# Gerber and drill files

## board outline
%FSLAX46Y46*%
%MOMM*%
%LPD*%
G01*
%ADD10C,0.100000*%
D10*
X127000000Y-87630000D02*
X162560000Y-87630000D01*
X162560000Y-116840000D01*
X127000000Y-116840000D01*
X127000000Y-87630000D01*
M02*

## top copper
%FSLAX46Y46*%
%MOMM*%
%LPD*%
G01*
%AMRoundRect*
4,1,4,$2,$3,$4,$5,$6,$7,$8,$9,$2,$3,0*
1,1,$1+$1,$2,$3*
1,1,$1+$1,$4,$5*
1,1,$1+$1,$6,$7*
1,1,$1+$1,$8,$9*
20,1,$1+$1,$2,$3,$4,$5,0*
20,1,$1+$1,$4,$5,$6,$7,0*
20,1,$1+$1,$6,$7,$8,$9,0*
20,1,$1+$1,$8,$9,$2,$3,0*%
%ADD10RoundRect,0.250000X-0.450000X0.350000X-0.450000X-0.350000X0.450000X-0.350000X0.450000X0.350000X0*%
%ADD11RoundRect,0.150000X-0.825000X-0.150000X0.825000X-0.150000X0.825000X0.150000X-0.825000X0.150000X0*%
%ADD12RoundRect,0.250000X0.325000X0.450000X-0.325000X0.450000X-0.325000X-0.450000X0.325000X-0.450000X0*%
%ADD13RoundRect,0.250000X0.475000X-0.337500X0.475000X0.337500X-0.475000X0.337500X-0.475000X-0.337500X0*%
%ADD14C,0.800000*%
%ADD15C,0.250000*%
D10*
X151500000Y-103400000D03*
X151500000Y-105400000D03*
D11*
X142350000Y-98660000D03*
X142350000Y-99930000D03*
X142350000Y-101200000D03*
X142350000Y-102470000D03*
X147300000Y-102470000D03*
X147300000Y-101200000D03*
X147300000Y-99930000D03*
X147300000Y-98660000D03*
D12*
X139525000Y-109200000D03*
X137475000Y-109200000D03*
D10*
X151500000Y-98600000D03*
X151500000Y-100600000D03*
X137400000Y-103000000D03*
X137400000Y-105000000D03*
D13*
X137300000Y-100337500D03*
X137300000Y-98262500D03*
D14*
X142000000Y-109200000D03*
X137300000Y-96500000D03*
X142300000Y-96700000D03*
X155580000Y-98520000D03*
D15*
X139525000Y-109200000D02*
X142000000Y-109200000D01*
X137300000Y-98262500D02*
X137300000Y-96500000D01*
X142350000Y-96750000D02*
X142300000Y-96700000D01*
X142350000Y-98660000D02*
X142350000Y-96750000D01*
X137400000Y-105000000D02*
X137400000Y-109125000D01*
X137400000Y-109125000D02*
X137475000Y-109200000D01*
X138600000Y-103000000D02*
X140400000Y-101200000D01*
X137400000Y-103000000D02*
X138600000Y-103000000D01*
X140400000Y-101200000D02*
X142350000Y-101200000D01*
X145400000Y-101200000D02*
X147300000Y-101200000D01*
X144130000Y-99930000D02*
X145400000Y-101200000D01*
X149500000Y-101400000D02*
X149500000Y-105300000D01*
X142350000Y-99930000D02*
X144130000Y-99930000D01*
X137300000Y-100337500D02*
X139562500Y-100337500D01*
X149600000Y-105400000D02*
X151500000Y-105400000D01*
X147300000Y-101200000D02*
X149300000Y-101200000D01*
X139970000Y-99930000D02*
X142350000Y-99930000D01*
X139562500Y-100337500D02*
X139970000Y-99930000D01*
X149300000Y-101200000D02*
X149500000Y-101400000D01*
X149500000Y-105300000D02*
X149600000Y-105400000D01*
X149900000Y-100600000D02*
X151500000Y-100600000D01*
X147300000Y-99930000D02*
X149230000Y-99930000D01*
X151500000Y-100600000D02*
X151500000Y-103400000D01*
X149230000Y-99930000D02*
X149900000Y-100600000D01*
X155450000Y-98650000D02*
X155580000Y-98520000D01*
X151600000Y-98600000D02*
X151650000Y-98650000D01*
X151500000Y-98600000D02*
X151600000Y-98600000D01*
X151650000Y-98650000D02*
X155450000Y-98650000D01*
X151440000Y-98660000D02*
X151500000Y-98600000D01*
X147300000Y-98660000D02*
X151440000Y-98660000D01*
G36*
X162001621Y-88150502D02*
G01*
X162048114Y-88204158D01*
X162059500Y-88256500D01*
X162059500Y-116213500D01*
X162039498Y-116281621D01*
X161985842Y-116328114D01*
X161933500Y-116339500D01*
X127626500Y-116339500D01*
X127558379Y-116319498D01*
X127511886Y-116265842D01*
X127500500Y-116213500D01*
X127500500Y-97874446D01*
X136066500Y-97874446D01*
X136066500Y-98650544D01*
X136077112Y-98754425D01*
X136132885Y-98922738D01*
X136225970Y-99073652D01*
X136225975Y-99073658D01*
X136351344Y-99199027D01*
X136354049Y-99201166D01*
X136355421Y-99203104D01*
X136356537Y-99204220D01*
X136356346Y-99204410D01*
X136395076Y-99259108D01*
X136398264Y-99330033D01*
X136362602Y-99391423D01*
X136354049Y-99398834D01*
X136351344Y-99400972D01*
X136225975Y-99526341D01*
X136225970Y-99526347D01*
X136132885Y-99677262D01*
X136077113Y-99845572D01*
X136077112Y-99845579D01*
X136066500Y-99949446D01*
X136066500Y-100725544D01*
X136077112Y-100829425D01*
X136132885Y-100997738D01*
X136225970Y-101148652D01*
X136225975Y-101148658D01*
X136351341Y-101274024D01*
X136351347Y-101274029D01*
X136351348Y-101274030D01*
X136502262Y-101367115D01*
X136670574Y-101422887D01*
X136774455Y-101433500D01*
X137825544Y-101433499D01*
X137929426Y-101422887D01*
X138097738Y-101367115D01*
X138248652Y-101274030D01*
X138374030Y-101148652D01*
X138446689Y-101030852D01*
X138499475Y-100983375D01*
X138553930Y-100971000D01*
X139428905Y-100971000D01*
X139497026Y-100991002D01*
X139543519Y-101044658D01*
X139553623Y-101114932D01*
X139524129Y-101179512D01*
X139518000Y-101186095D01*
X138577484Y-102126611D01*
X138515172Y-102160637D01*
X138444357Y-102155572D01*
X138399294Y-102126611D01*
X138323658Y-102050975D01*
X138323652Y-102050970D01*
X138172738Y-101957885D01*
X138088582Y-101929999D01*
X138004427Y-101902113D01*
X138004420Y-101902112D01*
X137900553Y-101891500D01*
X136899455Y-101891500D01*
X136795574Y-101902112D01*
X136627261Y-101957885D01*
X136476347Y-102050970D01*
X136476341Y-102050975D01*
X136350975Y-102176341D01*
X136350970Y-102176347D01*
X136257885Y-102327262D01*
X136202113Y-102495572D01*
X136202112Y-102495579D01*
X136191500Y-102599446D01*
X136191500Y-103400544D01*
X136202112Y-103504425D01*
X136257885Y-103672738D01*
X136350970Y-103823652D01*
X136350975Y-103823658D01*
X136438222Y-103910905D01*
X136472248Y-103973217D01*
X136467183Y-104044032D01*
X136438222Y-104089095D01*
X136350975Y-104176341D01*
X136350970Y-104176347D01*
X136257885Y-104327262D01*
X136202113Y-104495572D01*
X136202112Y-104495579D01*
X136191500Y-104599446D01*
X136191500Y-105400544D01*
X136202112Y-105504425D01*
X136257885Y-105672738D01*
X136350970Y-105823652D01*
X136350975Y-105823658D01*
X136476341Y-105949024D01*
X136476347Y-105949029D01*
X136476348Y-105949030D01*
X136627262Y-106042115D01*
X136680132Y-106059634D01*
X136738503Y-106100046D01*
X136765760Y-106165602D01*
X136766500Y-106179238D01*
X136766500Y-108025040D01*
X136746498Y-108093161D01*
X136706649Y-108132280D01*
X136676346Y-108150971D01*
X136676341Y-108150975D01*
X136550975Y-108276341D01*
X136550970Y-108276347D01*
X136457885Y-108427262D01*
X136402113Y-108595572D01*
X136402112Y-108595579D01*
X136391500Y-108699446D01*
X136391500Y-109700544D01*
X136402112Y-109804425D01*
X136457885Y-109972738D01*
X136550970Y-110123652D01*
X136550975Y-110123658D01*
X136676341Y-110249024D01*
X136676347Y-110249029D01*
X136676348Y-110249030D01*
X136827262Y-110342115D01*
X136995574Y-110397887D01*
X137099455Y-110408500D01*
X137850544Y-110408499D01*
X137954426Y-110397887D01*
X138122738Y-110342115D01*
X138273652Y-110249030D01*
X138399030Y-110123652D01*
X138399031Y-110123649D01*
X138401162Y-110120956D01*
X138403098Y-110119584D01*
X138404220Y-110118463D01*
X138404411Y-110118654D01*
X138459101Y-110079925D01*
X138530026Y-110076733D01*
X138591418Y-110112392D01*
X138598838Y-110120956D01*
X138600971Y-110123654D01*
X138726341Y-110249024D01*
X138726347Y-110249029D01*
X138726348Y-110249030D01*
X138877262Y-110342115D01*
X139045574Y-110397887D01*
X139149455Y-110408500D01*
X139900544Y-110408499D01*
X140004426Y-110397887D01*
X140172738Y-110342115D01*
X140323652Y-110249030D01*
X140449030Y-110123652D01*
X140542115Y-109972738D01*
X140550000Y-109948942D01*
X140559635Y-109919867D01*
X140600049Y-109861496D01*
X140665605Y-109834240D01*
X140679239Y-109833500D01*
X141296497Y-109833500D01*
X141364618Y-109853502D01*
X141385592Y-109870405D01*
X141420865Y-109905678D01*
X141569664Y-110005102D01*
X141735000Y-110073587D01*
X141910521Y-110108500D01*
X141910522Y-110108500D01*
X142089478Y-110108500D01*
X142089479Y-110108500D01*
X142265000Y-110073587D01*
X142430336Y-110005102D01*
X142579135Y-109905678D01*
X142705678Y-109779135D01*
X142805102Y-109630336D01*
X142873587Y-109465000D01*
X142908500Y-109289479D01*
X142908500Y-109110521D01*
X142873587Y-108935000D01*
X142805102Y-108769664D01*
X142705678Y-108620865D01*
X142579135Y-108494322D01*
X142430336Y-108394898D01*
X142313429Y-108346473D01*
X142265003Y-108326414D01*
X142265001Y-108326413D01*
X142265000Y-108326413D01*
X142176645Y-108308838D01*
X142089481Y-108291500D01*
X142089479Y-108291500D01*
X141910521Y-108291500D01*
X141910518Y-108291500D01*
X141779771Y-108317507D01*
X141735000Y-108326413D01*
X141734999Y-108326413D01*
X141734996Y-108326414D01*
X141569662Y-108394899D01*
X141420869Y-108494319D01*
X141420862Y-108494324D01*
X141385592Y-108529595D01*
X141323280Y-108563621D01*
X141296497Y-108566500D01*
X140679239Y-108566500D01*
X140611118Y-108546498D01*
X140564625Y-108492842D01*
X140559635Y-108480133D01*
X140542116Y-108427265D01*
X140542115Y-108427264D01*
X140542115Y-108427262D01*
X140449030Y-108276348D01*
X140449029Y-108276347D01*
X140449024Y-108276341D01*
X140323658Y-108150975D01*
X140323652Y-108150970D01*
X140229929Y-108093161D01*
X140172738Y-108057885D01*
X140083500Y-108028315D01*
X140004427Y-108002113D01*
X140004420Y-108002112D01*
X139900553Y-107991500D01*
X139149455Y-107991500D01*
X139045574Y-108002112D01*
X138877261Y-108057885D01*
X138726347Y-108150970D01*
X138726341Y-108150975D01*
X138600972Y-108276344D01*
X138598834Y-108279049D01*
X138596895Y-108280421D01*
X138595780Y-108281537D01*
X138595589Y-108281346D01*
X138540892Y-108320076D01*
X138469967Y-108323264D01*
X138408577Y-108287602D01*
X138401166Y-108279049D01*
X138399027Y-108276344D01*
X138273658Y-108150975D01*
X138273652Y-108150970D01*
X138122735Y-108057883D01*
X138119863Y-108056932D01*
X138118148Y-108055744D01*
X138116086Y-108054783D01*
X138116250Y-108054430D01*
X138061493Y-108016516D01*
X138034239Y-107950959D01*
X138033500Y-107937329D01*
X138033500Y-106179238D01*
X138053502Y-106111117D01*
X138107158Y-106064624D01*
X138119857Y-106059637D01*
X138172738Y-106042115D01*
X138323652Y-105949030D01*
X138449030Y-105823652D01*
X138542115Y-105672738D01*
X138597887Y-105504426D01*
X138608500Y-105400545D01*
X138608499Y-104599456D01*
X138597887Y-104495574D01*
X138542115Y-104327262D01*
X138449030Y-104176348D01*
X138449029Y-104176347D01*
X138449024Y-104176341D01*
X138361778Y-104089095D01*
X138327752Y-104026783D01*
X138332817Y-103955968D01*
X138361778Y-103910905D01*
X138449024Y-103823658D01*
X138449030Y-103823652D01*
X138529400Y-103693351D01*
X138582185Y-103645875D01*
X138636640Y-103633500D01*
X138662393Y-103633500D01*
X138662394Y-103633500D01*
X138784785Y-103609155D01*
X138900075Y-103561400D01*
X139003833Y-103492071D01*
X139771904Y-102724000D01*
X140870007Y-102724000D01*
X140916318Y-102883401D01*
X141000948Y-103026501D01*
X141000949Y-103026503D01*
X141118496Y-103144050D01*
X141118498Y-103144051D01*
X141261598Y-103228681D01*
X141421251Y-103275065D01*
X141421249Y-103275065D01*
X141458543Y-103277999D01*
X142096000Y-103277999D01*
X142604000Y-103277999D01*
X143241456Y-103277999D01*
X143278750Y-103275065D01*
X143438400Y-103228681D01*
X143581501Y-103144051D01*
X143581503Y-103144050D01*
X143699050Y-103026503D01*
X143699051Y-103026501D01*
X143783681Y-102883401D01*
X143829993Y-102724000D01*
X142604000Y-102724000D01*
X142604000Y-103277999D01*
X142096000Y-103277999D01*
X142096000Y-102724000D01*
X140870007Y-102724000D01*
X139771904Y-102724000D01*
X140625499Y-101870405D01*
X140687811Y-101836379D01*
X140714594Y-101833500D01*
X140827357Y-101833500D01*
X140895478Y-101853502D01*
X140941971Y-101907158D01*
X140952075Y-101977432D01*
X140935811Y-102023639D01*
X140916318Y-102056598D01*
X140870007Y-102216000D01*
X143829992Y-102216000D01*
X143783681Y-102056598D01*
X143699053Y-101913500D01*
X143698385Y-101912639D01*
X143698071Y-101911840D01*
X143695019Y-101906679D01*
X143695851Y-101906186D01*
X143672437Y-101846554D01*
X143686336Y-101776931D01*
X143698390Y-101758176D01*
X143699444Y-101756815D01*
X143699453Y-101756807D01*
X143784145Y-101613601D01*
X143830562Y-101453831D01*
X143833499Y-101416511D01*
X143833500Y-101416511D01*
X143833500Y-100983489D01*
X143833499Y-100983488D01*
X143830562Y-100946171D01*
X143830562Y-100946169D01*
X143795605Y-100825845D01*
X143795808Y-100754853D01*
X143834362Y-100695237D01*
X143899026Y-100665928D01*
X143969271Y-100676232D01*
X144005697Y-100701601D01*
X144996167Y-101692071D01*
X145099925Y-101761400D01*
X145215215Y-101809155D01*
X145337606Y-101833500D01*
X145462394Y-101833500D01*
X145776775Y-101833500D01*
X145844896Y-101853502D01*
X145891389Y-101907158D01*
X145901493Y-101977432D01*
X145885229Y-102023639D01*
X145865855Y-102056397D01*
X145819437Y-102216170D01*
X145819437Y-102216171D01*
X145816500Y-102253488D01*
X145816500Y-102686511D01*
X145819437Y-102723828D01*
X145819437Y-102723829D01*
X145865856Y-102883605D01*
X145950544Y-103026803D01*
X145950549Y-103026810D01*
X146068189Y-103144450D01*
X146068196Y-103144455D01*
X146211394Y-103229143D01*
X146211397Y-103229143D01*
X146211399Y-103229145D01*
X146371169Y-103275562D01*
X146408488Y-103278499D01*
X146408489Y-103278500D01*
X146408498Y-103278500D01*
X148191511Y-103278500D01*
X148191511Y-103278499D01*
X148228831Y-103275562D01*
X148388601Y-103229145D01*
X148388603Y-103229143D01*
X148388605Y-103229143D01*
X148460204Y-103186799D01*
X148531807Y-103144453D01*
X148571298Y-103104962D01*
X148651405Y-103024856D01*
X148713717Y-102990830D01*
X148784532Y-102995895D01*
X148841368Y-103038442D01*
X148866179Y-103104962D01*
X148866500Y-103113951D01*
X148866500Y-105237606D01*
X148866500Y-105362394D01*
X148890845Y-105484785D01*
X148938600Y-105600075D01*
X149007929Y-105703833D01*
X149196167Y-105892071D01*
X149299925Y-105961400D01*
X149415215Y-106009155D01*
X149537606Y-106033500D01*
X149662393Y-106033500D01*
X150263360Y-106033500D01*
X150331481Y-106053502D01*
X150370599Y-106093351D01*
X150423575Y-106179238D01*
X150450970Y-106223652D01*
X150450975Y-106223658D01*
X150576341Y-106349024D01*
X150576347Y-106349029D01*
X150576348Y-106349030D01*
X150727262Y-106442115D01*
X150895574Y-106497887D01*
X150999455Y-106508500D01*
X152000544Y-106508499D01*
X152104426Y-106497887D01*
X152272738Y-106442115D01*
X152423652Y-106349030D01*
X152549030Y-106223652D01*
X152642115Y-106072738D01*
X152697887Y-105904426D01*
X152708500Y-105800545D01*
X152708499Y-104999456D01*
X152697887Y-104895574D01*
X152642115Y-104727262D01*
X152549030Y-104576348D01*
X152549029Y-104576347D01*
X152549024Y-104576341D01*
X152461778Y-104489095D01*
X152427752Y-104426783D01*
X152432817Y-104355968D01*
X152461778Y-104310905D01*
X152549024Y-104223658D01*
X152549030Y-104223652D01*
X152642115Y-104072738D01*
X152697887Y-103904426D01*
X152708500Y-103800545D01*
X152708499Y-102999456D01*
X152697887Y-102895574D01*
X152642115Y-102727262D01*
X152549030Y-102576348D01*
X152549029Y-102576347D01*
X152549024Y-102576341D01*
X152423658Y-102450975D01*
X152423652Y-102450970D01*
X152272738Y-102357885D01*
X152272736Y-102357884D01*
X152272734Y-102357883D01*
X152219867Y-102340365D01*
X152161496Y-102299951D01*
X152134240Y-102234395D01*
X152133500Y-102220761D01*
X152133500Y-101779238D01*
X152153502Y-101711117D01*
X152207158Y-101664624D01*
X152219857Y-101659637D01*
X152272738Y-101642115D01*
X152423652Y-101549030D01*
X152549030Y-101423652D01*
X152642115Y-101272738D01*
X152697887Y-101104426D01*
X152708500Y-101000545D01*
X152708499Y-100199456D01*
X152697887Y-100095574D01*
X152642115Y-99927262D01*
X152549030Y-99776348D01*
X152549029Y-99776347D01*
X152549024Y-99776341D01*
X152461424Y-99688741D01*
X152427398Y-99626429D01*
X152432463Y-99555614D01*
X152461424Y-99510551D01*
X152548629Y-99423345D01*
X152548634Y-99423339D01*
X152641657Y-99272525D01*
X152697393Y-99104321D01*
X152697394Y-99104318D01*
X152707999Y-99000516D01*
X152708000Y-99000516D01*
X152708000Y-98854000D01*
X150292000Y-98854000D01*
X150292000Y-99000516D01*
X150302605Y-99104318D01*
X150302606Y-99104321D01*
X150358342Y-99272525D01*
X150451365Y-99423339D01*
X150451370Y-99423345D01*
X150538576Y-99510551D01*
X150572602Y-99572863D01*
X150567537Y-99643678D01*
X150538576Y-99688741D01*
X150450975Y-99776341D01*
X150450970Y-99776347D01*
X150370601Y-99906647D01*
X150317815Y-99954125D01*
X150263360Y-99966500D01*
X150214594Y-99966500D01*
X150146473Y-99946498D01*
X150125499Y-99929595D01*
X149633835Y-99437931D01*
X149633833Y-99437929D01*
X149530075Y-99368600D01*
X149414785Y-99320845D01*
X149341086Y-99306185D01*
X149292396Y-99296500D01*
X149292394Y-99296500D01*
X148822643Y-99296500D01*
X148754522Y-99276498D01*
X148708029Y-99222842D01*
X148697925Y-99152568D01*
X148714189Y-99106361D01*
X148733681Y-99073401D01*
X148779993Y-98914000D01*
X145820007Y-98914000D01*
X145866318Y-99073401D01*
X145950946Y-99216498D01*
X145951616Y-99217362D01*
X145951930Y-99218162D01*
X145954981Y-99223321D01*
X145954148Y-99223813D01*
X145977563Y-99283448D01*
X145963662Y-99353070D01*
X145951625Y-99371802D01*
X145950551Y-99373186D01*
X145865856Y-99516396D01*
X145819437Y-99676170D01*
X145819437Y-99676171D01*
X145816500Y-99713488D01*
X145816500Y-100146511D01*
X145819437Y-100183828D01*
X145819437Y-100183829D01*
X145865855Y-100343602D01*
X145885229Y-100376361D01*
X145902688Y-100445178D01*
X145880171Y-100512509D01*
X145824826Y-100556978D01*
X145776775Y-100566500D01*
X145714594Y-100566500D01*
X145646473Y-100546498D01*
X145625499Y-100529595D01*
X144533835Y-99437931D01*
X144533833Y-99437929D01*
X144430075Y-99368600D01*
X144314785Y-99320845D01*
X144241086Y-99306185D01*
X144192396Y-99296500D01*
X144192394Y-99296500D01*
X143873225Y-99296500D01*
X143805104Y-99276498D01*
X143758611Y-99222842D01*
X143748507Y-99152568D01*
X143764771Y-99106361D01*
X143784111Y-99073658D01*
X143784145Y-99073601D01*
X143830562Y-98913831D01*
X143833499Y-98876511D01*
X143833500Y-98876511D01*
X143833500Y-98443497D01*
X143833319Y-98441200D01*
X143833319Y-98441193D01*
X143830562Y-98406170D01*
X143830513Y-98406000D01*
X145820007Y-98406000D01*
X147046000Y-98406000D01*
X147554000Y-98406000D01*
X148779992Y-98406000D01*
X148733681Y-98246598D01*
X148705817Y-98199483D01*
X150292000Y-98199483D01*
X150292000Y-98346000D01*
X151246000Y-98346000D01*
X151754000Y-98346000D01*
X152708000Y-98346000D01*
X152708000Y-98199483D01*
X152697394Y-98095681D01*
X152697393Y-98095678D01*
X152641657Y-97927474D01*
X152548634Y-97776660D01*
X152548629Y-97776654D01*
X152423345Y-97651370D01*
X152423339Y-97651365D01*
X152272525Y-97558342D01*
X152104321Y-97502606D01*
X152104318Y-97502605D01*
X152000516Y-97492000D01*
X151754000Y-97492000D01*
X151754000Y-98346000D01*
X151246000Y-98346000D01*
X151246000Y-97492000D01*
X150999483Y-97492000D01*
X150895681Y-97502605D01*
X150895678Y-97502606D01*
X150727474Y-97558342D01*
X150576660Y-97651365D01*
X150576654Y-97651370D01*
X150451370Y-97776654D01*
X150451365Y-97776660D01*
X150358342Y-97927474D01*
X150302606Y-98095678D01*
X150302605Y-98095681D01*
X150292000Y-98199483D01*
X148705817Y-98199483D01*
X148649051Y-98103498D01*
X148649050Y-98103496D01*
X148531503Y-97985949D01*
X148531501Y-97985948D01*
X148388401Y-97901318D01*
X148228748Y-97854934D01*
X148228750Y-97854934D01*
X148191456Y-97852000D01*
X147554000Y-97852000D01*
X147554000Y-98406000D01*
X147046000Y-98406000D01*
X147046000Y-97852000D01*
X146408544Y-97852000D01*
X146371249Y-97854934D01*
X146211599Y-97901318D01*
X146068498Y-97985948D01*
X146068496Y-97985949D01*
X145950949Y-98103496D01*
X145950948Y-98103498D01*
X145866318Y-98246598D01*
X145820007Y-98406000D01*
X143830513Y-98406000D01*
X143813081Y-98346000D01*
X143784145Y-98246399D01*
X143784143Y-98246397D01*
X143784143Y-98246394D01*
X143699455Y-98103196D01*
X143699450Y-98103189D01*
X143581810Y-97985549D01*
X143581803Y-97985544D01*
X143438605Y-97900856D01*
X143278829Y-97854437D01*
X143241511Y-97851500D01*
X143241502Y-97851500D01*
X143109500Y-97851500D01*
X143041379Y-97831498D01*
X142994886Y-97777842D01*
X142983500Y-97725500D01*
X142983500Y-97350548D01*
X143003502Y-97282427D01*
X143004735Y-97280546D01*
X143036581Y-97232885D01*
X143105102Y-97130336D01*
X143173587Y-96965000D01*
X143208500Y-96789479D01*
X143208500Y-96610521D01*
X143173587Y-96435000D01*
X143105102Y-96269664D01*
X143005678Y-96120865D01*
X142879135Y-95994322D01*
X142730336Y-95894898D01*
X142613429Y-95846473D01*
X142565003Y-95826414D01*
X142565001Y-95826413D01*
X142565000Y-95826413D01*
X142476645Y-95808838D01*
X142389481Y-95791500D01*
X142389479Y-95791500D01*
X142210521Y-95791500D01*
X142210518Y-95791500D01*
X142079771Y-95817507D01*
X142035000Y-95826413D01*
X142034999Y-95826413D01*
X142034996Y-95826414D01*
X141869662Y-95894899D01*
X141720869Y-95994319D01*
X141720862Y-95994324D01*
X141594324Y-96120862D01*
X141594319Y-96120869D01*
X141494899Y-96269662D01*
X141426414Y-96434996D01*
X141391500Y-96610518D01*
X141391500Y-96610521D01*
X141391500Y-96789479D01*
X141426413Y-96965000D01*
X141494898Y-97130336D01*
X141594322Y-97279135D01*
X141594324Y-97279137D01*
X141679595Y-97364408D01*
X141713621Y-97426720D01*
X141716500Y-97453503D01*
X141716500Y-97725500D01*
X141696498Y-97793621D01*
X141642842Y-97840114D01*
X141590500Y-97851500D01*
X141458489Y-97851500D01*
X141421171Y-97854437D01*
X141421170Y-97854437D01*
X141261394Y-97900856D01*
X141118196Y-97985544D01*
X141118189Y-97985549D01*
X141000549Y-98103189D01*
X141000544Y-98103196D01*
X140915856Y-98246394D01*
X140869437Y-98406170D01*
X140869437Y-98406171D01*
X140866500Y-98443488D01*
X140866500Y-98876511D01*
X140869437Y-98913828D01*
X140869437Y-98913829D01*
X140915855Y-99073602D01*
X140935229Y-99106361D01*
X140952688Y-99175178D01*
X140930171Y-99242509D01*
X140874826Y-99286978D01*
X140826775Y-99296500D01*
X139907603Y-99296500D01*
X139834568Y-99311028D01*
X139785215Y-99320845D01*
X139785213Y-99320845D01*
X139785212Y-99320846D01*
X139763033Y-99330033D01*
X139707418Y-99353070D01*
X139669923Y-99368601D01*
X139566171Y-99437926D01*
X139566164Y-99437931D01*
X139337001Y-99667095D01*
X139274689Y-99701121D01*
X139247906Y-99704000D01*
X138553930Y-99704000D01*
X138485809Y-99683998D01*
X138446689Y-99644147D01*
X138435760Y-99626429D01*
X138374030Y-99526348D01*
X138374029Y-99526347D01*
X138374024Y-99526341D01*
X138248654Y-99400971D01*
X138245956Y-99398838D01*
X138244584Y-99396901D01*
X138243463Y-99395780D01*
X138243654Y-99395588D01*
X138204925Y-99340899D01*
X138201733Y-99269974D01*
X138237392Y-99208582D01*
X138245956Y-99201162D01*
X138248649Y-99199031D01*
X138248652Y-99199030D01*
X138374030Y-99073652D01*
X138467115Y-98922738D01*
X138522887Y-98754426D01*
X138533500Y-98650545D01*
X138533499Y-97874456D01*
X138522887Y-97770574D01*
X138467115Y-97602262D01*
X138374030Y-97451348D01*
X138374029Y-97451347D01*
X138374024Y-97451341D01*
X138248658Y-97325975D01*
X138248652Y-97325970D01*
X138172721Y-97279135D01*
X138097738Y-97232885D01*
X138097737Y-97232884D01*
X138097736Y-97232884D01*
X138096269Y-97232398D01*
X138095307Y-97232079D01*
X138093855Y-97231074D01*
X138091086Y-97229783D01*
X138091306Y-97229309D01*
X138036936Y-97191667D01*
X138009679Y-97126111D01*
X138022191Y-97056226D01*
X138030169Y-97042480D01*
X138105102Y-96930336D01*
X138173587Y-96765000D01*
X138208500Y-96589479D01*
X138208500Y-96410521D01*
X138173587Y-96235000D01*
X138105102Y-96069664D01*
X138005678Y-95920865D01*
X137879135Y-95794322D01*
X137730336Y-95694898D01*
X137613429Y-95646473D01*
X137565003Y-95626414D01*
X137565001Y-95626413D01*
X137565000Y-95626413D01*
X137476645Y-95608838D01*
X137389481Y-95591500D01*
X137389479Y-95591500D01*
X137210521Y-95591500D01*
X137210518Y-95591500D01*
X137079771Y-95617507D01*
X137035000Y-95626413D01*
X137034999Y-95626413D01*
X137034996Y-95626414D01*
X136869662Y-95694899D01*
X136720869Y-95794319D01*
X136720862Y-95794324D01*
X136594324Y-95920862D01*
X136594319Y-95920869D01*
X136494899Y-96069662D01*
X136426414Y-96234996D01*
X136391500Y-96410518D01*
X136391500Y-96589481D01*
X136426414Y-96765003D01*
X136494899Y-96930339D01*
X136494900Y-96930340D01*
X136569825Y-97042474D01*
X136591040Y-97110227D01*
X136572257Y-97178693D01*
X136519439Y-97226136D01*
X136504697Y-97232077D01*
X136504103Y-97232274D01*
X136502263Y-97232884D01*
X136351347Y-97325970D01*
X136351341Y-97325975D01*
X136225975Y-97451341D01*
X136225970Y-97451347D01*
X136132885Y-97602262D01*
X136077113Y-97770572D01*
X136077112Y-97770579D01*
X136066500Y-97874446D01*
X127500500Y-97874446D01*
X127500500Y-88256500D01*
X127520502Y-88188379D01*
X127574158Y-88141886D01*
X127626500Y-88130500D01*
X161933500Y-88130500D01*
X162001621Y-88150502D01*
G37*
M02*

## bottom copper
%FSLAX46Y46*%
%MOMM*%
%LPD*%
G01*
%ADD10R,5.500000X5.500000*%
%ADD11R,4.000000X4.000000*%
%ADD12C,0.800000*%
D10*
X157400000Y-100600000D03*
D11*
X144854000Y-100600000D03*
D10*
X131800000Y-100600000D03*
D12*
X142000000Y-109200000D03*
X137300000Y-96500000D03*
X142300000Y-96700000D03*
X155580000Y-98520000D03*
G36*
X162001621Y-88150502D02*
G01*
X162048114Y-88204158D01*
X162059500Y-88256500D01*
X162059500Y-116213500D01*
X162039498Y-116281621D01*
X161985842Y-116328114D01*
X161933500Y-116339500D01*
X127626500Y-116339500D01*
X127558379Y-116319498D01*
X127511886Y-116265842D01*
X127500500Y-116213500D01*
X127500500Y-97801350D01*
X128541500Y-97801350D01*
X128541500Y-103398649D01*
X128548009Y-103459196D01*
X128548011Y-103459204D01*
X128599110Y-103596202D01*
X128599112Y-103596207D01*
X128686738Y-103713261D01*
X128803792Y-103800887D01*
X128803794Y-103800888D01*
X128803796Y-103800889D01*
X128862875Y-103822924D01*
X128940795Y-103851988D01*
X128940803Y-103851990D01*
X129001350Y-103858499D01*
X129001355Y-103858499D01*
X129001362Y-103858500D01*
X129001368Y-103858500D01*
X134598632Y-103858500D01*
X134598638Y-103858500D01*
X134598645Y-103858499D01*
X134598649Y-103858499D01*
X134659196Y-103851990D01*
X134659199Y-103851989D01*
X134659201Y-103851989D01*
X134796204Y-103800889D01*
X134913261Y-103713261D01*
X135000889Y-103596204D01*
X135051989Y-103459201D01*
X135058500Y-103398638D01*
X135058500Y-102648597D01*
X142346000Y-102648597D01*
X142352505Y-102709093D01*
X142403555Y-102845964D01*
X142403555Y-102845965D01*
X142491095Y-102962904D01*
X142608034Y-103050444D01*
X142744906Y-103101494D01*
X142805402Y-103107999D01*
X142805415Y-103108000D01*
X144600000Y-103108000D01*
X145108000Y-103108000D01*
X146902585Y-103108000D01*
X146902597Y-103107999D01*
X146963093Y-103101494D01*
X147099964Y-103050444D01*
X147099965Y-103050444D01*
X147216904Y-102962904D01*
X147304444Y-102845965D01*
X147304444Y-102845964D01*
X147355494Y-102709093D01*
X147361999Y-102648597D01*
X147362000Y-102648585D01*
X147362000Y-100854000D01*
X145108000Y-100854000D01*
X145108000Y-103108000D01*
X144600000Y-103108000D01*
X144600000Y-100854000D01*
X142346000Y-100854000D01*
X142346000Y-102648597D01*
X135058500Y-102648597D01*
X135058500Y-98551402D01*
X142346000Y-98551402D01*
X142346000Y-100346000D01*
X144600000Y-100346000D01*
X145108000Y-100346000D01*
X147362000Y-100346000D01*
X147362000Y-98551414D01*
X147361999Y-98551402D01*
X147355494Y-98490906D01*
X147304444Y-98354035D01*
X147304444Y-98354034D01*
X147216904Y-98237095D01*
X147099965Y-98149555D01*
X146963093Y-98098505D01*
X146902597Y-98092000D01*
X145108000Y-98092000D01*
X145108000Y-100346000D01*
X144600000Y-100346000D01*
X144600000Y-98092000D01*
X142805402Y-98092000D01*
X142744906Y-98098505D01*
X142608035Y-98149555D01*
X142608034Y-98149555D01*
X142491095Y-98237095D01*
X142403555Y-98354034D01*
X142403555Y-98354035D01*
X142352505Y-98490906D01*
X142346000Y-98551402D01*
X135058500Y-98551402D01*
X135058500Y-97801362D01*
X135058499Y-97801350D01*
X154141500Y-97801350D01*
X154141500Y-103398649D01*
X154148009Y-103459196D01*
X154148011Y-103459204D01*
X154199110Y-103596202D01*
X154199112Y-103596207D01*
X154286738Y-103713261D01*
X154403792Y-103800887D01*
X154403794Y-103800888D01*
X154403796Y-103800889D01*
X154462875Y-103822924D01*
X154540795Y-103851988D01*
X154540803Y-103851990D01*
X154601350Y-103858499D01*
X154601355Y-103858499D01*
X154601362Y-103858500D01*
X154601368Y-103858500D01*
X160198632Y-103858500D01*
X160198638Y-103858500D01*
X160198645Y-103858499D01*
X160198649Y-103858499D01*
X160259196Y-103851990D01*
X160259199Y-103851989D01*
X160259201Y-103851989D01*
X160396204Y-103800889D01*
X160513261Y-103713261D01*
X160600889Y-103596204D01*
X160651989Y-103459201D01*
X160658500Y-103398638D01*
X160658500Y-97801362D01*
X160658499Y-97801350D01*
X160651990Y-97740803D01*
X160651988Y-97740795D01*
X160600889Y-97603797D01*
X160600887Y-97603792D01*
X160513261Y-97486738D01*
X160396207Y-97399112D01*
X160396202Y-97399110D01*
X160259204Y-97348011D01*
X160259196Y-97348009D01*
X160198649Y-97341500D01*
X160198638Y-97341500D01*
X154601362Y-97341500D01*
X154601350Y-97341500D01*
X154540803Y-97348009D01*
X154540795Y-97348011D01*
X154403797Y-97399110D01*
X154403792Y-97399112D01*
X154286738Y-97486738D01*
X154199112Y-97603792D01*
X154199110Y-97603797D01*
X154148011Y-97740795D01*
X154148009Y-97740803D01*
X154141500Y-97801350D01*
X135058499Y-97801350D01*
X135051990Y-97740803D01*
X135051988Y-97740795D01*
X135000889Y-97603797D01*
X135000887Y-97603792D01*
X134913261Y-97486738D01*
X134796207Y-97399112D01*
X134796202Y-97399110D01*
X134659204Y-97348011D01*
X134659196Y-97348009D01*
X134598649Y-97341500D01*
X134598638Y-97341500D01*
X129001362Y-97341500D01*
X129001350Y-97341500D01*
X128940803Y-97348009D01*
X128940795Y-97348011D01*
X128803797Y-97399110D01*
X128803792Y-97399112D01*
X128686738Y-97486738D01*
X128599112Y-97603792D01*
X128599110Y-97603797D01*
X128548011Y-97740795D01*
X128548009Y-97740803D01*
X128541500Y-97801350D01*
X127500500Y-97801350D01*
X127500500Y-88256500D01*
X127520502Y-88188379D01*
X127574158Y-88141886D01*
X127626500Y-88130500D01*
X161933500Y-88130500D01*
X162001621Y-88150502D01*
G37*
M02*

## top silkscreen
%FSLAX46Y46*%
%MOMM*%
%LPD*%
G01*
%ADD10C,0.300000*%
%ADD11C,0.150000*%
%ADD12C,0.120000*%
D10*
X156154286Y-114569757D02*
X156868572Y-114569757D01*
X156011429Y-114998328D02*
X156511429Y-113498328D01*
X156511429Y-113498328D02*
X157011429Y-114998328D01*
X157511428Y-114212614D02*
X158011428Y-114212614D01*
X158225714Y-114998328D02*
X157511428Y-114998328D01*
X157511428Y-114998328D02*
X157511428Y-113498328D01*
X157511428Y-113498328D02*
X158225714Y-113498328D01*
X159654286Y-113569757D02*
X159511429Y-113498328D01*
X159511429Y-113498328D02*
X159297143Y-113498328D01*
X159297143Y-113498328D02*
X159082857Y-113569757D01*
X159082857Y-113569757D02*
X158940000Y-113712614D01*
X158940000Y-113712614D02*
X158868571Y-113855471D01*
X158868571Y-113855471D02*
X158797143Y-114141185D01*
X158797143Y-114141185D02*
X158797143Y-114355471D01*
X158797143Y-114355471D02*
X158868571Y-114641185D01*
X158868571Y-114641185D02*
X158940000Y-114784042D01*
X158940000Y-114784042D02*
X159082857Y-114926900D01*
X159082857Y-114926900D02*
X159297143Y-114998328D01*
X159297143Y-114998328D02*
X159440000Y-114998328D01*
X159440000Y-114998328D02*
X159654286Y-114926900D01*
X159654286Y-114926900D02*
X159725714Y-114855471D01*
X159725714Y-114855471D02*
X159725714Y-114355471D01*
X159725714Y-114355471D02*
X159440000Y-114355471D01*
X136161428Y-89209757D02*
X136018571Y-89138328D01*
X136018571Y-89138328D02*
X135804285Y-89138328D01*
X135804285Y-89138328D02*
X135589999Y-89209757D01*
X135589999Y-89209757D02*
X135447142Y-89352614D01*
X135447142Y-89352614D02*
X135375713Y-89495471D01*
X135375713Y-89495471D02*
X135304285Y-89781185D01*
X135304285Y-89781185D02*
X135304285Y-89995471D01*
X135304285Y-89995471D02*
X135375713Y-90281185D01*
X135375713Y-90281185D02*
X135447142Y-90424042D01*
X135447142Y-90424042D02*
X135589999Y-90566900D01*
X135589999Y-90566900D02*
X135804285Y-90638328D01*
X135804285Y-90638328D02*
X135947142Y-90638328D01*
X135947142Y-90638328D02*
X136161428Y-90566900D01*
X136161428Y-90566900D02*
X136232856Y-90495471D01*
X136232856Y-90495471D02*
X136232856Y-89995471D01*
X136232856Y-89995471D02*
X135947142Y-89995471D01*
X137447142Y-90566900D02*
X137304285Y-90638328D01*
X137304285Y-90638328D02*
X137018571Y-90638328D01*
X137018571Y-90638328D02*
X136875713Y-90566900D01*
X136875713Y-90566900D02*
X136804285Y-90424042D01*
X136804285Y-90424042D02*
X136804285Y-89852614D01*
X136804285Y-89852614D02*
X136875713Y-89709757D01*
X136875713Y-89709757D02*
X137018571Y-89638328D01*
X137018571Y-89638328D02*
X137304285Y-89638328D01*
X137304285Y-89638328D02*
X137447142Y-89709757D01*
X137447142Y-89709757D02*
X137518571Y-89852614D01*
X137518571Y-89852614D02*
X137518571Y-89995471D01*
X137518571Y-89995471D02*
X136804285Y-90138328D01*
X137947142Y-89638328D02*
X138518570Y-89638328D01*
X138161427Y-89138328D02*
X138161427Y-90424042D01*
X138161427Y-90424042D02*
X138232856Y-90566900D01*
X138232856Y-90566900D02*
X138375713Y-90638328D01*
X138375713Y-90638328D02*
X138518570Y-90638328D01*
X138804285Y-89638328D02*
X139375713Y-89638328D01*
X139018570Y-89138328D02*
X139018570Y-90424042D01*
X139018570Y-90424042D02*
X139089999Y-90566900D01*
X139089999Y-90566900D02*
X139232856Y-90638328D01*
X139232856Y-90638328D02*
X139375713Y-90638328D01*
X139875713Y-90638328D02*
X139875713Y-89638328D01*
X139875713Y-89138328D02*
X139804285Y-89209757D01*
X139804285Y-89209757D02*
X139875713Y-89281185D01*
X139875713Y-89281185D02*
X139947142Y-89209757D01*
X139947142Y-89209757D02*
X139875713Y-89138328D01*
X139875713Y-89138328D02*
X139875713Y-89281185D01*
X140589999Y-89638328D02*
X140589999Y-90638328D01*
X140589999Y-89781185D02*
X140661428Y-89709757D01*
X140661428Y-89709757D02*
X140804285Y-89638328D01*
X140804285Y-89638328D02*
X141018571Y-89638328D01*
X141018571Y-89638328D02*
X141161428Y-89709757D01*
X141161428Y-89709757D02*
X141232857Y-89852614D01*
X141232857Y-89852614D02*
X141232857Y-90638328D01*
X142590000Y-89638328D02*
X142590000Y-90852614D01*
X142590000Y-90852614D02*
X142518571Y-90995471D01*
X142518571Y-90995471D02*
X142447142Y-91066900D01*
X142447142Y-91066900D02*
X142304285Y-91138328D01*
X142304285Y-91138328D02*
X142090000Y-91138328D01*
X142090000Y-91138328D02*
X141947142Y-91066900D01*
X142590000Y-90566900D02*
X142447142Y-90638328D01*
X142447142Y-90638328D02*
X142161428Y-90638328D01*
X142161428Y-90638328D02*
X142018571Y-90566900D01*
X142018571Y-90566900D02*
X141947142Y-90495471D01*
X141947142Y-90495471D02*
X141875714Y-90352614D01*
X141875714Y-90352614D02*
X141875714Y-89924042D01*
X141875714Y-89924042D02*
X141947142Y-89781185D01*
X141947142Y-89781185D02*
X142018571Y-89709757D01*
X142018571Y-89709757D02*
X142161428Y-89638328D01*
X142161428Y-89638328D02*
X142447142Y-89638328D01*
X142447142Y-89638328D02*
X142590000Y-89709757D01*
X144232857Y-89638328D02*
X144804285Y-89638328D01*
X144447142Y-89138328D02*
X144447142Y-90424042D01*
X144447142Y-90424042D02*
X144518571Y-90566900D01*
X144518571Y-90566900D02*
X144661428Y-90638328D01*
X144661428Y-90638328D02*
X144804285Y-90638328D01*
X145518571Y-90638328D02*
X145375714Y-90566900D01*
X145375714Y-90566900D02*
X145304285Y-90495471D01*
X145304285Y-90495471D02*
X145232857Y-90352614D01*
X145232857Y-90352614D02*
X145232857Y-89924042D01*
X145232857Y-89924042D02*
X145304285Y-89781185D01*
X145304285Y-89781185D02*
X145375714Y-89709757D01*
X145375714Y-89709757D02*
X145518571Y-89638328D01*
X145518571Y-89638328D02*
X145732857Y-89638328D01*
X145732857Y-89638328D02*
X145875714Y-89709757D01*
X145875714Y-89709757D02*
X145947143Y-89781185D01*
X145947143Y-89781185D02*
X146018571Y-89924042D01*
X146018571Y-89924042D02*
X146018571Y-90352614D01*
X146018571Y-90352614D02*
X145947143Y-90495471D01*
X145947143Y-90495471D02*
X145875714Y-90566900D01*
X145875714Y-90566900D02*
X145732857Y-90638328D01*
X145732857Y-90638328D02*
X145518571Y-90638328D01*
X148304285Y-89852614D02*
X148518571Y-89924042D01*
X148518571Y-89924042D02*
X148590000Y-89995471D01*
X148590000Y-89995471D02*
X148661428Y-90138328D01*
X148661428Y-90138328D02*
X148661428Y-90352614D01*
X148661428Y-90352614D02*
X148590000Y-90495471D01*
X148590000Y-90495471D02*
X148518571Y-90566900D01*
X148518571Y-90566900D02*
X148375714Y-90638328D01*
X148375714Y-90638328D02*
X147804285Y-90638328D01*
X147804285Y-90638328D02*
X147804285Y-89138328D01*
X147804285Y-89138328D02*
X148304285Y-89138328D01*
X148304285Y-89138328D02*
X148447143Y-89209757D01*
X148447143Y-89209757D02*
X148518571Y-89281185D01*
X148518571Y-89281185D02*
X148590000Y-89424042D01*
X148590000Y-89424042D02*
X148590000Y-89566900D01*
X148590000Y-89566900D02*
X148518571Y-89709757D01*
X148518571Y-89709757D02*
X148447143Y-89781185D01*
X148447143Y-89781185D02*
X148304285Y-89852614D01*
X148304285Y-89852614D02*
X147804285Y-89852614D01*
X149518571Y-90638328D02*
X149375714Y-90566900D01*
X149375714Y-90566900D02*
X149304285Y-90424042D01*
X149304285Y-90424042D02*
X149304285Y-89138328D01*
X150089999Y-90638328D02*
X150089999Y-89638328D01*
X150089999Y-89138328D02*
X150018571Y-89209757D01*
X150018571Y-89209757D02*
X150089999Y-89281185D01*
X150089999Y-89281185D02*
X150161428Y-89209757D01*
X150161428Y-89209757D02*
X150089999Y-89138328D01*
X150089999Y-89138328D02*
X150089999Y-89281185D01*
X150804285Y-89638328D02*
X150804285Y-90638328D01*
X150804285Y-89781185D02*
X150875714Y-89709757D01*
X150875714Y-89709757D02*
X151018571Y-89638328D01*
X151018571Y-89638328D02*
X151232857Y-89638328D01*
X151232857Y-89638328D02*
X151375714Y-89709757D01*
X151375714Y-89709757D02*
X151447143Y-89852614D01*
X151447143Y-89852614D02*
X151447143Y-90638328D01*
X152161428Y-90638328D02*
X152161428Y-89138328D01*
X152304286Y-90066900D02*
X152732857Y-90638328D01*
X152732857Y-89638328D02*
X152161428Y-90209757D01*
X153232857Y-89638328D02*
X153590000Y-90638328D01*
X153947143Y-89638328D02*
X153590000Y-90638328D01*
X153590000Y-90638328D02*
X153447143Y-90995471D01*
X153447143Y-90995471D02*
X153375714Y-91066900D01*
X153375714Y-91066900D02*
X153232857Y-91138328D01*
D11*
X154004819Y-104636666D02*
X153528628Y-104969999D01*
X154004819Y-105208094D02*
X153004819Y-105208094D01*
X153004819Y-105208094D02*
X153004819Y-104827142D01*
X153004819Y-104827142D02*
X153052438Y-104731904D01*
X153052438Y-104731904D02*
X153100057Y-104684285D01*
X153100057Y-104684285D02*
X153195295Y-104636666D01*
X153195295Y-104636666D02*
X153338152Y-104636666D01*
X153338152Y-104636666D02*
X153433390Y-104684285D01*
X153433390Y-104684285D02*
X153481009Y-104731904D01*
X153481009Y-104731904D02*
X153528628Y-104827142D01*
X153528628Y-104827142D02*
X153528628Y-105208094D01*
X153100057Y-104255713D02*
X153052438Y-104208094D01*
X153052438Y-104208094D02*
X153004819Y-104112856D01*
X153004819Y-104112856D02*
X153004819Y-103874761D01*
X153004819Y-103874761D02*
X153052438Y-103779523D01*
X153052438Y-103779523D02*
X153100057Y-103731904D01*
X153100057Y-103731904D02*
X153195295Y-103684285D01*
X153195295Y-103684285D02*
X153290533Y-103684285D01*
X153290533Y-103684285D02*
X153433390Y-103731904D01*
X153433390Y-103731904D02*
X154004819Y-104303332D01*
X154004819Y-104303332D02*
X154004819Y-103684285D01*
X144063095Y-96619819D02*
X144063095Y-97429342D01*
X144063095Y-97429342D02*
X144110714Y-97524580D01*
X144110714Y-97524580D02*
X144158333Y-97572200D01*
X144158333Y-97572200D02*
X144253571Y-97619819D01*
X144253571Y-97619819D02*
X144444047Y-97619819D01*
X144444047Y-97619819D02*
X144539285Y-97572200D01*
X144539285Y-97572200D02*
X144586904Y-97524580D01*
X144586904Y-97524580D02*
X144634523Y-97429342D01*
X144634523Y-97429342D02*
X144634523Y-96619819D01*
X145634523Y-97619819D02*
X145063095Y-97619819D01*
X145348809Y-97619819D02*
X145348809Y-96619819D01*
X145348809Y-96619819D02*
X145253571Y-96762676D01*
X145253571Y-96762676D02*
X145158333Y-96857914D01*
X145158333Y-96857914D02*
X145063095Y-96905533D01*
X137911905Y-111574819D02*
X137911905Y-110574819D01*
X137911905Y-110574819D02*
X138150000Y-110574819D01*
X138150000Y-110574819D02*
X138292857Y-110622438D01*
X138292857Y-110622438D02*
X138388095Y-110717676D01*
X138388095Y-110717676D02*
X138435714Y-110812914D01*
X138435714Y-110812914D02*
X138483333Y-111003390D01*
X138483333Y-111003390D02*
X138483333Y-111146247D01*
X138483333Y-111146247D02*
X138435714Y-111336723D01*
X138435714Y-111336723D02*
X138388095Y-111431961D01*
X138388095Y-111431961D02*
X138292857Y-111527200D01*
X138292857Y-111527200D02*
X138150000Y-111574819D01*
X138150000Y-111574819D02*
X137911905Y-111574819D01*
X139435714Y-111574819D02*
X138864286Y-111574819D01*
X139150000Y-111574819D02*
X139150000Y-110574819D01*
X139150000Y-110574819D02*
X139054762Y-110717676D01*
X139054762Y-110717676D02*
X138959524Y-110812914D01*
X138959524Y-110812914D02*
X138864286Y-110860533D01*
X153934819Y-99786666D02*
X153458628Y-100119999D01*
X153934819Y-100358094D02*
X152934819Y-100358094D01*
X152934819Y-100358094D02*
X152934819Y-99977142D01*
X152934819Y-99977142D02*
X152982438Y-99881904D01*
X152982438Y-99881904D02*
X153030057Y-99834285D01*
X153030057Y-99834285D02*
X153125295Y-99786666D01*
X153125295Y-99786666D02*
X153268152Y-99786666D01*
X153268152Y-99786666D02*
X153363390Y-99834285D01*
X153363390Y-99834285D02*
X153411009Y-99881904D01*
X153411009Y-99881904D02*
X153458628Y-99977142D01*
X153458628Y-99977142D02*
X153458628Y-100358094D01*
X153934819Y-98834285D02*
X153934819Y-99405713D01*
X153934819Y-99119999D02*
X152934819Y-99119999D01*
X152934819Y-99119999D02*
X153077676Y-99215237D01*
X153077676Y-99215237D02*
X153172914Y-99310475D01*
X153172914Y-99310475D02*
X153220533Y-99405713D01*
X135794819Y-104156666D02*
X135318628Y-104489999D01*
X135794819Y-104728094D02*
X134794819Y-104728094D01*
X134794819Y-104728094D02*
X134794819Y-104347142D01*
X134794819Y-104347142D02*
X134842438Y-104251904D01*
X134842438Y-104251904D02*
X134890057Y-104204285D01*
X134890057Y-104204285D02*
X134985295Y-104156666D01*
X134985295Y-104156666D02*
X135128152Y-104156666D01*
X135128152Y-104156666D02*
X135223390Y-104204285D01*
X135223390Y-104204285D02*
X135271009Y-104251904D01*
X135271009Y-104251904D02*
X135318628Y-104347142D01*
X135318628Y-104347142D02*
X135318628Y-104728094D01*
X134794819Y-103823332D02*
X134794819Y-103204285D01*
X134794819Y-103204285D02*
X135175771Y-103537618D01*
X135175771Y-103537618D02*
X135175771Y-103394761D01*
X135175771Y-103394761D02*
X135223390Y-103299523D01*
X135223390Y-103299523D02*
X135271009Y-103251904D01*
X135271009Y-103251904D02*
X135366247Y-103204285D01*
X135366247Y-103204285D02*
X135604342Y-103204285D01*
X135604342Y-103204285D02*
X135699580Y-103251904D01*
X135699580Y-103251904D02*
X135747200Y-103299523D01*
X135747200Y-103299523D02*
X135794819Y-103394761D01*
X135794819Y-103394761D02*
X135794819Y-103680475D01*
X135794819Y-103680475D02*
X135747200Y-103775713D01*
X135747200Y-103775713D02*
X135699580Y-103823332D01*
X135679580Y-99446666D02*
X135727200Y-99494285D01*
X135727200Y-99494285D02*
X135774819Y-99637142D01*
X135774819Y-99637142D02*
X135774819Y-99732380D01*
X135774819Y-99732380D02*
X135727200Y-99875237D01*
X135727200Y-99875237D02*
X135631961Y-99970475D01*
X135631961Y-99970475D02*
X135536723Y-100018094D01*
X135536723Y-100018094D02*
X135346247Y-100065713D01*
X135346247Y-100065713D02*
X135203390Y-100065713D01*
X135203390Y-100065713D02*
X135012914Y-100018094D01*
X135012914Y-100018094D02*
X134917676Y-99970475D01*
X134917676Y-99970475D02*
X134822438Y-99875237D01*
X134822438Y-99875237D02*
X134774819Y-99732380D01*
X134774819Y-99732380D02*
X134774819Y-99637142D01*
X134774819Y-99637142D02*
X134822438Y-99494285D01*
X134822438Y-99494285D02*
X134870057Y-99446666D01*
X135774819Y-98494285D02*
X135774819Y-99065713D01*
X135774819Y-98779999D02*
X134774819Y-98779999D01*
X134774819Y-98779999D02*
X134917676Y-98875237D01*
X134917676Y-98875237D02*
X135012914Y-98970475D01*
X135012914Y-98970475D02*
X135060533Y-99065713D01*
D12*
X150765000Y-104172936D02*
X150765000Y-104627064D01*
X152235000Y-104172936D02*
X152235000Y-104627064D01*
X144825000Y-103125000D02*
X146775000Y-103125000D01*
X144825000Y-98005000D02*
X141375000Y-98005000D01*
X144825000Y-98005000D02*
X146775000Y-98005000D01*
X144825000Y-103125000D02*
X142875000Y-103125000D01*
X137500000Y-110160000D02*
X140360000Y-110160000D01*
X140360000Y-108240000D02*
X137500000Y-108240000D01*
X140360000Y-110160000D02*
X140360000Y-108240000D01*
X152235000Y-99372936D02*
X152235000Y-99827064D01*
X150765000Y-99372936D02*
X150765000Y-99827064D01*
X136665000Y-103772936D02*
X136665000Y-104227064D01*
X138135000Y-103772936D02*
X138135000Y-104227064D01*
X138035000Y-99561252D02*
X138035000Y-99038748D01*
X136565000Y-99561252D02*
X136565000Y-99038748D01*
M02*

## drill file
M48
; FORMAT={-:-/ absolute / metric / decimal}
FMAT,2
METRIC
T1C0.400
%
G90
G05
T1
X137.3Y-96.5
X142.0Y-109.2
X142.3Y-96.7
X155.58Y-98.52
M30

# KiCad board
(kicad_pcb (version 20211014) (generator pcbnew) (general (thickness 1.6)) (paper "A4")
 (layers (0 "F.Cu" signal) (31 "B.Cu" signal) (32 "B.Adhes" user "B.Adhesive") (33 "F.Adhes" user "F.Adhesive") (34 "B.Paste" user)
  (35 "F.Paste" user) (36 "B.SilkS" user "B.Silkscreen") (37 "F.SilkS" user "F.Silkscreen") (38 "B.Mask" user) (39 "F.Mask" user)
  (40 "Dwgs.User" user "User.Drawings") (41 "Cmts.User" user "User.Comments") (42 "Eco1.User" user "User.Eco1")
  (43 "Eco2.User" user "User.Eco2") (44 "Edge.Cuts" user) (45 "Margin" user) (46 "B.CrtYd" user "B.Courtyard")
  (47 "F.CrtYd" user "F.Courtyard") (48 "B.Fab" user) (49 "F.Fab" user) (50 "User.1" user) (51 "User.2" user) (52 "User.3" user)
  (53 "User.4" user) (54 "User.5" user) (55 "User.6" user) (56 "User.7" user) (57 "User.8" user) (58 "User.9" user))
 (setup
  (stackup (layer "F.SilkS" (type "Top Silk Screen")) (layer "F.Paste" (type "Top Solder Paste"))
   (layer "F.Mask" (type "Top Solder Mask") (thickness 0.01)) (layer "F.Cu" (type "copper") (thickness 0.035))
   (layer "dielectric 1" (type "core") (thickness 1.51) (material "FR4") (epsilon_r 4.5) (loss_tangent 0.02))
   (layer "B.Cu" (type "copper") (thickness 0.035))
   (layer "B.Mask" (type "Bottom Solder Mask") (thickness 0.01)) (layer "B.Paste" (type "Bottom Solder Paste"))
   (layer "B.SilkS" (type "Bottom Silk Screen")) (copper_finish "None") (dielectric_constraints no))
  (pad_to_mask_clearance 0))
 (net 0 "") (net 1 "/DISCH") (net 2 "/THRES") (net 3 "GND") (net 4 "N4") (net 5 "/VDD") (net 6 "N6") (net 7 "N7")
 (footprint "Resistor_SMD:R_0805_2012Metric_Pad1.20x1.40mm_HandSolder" (layer "F.Cu") (at 151.5 104.4 -90)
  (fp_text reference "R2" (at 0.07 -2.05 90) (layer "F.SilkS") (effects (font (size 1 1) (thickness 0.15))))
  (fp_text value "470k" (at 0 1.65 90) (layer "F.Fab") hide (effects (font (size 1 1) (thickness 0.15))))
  (fp_line (start -0.227064 0.735) (end 0.227064 0.735) (layer "F.SilkS") (width 0.12))
  (fp_line (start -0.227064 -0.735) (end 0.227064 -0.735) (layer "F.SilkS") (width 0.12))
  (pad "1" smd roundrect (at -1 0 270) (size 1.2 1.4) (layers "F.Cu" "F.Paste" "F.Mask") (roundrect_rratio 0.208333) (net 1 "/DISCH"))
  (pad "2" smd roundrect (at 1 0 270) (size 1.2 1.4) (layers "F.Cu" "F.Paste" "F.Mask") (roundrect_rratio 0.208333) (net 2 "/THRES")))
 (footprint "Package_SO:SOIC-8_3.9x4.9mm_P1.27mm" (layer "F.Cu") (at 144.825 100.565)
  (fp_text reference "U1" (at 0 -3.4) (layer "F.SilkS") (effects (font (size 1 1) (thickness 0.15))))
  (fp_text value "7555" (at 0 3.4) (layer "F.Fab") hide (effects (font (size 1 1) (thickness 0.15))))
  (fp_line (start 0 2.56) (end 1.95 2.56) (layer "F.SilkS") (width 0.12))
  (fp_line (start 0 -2.56) (end -3.45 -2.56) (layer "F.SilkS") (width 0.12))
  (fp_line (start 0 -2.56) (end 1.95 -2.56) (layer "F.SilkS") (width 0.12))
  (fp_line (start 0 2.56) (end -1.95 2.56) (layer "F.SilkS") (width 0.12))
  (pad "1" smd roundrect (at -2.475 -1.905) (size 1.95 0.6) (layers "F.Cu" "F.Paste" "F.Mask") (roundrect_rratio 0.25) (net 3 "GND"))
  (pad "2" smd roundrect (at -2.475 -0.635) (size 1.95 0.6) (layers "F.Cu" "F.Paste" "F.Mask") (roundrect_rratio 0.25) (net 2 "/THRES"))
  (pad "3" smd roundrect (at -2.475 0.635) (size 1.95 0.6) (layers "F.Cu" "F.Paste" "F.Mask") (roundrect_rratio 0.25) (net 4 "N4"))
  (pad "4" smd roundrect (at -2.475 1.905) (size 1.95 0.6) (layers "F.Cu" "F.Paste" "F.Mask") (roundrect_rratio 0.25) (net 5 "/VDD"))
  (pad "5" smd roundrect (at 2.475 1.905) (size 1.95 0.6) (layers "F.Cu" "F.Paste" "F.Mask") (roundrect_rratio 0.25) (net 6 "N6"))
  (pad "6" smd roundrect (at 2.475 0.635) (size 1.95 0.6) (layers "F.Cu" "F.Paste" "F.Mask") (roundrect_rratio 0.25) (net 2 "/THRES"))
  (pad "7" smd roundrect (at 2.475 -0.635) (size 1.95 0.6) (layers "F.Cu" "F.Paste" "F.Mask") (roundrect_rratio 0.25) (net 1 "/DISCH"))
  (pad "8" smd roundrect (at 2.475 -1.905) (size 1.95 0.6) (layers "F.Cu" "F.Paste" "F.Mask") (roundrect_rratio 0.25) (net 5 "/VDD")))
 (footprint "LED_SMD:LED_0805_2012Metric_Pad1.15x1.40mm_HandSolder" (layer "F.Cu") (at 138.5 109.2 180)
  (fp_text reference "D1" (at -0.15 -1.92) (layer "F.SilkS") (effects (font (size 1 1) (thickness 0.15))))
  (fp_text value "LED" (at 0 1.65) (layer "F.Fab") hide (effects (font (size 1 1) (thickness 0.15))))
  (fp_line (start 1 -0.96) (end -1.86 -0.96) (layer "F.SilkS") (width 0.12))
  (fp_line (start -1.86 0.96) (end 1 0.96) (layer "F.SilkS") (width 0.12))
  (fp_line (start -1.86 -0.96) (end -1.86 0.96) (layer "F.SilkS") (width 0.12))
  (pad "1" smd roundrect (at -1.025 0 180) (size 1.15 1.4) (layers "F.Cu" "F.Paste" "F.Mask") (roundrect_rratio 0.217391) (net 3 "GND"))
  (pad "2" smd roundrect (at 1.025 0 180) (size 1.15 1.4) (layers "F.Cu" "F.Paste" "F.Mask") (roundrect_rratio 0.217391) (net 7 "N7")))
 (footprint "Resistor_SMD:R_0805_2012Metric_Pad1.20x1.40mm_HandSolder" (layer "F.Cu") (at 151.5 99.6 -90)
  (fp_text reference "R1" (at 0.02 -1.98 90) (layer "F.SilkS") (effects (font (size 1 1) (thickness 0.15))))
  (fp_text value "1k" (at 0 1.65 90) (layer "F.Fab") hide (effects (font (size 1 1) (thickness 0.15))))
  (fp_line (start -0.227064 -0.735) (end 0.227064 -0.735) (layer "F.SilkS") (width 0.12))
  (fp_line (start -0.227064 0.735) (end 0.227064 0.735) (layer "F.SilkS") (width 0.12))
  (pad "1" smd roundrect (at -1 0 270) (size 1.2 1.4) (layers "F.Cu" "F.Paste" "F.Mask") (roundrect_rratio 0.208333) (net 5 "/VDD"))
  (pad "2" smd roundrect (at 1 0 270) (size 1.2 1.4) (layers "F.Cu" "F.Paste" "F.Mask") (roundrect_rratio 0.208333) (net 1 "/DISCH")))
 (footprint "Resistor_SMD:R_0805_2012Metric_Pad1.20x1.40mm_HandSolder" (layer "F.Cu") (at 137.4 104 -90)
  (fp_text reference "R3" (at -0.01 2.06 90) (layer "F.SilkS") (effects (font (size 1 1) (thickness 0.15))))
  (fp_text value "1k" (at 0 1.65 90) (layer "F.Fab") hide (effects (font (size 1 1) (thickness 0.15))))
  (fp_line (start -0.227064 0.735) (end 0.227064 0.735) (layer "F.SilkS") (width 0.12))
  (fp_line (start -0.227064 -0.735) (end 0.227064 -0.735) (layer "F.SilkS") (width 0.12))
  (pad "1" smd roundrect (at -1 0 270) (size 1.2 1.4) (layers "F.Cu" "F.Paste" "F.Mask") (roundrect_rratio 0.208333) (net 4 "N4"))
  (pad "2" smd roundrect (at 1 0 270) (size 1.2 1.4) (layers "F.Cu" "F.Paste" "F.Mask") (roundrect_rratio 0.208333) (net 7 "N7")))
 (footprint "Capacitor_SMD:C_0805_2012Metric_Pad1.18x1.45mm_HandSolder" (layer "F.Cu") (at 137.3 99.3 90)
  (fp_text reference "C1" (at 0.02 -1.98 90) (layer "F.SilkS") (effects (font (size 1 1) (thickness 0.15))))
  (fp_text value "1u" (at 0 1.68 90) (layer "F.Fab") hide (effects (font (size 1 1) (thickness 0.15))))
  (fp_line (start -0.261252 0.735) (end 0.261252 0.735) (layer "F.SilkS") (width 0.12))
  (fp_line (start -0.261252 -0.735) (end 0.261252 -0.735) (layer "F.SilkS") (width 0.12))
  (pad "1" smd roundrect (at -1.0375 0 90) (size 1.175 1.45) (layers "F.Cu" "F.Paste" "F.Mask") (roundrect_rratio 0.212766) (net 2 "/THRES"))
  (pad "2" smd roundrect (at 1.0375 0 90) (size 1.175 1.45) (layers "F.Cu" "F.Paste" "F.Mask") (roundrect_rratio 0.212766) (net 3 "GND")))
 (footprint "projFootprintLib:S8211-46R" (layer "B.Cu") (at 144.6 100.6 180)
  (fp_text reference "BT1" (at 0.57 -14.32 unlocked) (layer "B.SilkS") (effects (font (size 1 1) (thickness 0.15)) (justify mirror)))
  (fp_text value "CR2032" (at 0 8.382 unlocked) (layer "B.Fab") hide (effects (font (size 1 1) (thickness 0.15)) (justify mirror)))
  (pad "1" smd rect (at -12.8 0 180) (size 5.5 5.5) (layers "B.Cu" "B.Paste" "B.Mask") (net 5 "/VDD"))
  (pad "2" smd rect (at -0.254 0 180) (size 4 4) (layers "B.Cu" "B.Paste" "B.Mask") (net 3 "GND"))
  (pad "3" smd rect (at 12.8 0 180) (size 5.5 5.5) (layers "B.Cu" "B.Paste" "B.Mask")))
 (gr_rect (start 127 87.63) (end 162.56 116.84) (layer "Edge.Cuts") (width 0.1) (fill none))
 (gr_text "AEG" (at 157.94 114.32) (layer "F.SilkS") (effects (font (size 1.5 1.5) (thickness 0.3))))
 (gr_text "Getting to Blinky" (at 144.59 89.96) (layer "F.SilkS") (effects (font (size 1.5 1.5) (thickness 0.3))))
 (segment (start 139.525 109.2) (end 142 109.2) (width 0.25) (layer "F.Cu") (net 3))
 (segment (start 137.3 98.2625) (end 137.3 96.5) (width 0.25) (layer "F.Cu") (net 3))
 (segment (start 142.35 96.75) (end 142.3 96.7) (width 0.25) (layer "F.Cu") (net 3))
 (segment (start 142.35 98.66) (end 142.35 96.75) (width 0.25) (layer "F.Cu") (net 3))
 (via (at 142 109.2) (size 0.8) (drill 0.4) (layers "F.Cu" "B.Cu") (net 3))
 (via (at 137.3 96.5) (size 0.8) (drill 0.4) (layers "F.Cu" "B.Cu") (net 3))
 (via (at 142.3 96.7) (size 0.8) (drill 0.4) (layers "F.Cu" "B.Cu") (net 3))
 (segment (start 137.4 105) (end 137.4 109.125) (width 0.25) (layer "F.Cu") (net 7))
 (segment (start 137.4 109.125) (end 137.475 109.2) (width 0.25) (layer "F.Cu") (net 7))
 (segment (start 138.6 103) (end 140.4 101.2) (width 0.25) (layer "F.Cu") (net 4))
 (segment (start 137.4 103) (end 138.6 103) (width 0.25) (layer "F.Cu") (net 4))
 (segment (start 140.4 101.2) (end 142.35 101.2) (width 0.25) (layer "F.Cu") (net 4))
 (segment (start 145.4 101.2) (end 147.3 101.2) (width 0.25) (layer "F.Cu") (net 2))
 (segment (start 144.13 99.93) (end 145.4 101.2) (width 0.25) (layer "F.Cu") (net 2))
 (segment (start 149.5 101.4) (end 149.5 105.3) (width 0.25) (layer "F.Cu") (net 2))
 (segment (start 142.35 99.93) (end 144.13 99.93) (width 0.25) (layer "F.Cu") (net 2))
 (segment (start 137.3 100.3375) (end 139.5625 100.3375) (width 0.25) (layer "F.Cu") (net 2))
 (segment (start 149.6 105.4) (end 151.5 105.4) (width 0.25) (layer "F.Cu") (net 2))
 (segment (start 147.3 101.2) (end 149.3 101.2) (width 0.25) (layer "F.Cu") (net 2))
 (segment (start 139.97 99.93) (end 142.35 99.93) (width 0.25) (layer "F.Cu") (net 2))
 (segment (start 139.5625 100.3375) (end 139.97 99.93) (width 0.25) (layer "F.Cu") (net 2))
 (segment (start 149.3 101.2) (end 149.5 101.4) (width 0.25) (layer "F.Cu") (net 2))
 (segment (start 149.5 105.3) (end 149.6 105.4) (width 0.25) (layer "F.Cu") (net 2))
 (segment (start 149.9 100.6) (end 151.5 100.6) (width 0.25) (layer "F.Cu") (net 1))
 (segment (start 147.3 99.93) (end 149.23 99.93) (width 0.25) (layer "F.Cu") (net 1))
 (segment (start 151.5 100.6) (end 151.5 103.4) (width 0.25) (layer "F.Cu") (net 1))
 (segment (start 149.23 99.93) (end 149.9 100.6) (width 0.25) (layer "F.Cu") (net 1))
 (segment (start 155.45 98.65) (end 155.58 98.52) (width 0.25) (layer "F.Cu") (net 5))
 (segment (start 151.6 98.6) (end 151.65 98.65) (width 0.25) (layer "F.Cu") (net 5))
 (segment (start 151.5 98.6) (end 151.6 98.6) (width 0.25) (layer "F.Cu") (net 5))
 (segment (start 151.65 98.65) (end 155.45 98.65) (width 0.25) (layer "F.Cu") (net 5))
 (segment (start 151.44 98.66) (end 151.5 98.6) (width 0.25) (layer "F.Cu") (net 5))
 (segment (start 147.3 98.66) (end 151.44 98.66) (width 0.25) (layer "F.Cu") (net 5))
 (via (at 155.58 98.52) (size 0.8) (drill 0.4) (layers "F.Cu" "B.Cu") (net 5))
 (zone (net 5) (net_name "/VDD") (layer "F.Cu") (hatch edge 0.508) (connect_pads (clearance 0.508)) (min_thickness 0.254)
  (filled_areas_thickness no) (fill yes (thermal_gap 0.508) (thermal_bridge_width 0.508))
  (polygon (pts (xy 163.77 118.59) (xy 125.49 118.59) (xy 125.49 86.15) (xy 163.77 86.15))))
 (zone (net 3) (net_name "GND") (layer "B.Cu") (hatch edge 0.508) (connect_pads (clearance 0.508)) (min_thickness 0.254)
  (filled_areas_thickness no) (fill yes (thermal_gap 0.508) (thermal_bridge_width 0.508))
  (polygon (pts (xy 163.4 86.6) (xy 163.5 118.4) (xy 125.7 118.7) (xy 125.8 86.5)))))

